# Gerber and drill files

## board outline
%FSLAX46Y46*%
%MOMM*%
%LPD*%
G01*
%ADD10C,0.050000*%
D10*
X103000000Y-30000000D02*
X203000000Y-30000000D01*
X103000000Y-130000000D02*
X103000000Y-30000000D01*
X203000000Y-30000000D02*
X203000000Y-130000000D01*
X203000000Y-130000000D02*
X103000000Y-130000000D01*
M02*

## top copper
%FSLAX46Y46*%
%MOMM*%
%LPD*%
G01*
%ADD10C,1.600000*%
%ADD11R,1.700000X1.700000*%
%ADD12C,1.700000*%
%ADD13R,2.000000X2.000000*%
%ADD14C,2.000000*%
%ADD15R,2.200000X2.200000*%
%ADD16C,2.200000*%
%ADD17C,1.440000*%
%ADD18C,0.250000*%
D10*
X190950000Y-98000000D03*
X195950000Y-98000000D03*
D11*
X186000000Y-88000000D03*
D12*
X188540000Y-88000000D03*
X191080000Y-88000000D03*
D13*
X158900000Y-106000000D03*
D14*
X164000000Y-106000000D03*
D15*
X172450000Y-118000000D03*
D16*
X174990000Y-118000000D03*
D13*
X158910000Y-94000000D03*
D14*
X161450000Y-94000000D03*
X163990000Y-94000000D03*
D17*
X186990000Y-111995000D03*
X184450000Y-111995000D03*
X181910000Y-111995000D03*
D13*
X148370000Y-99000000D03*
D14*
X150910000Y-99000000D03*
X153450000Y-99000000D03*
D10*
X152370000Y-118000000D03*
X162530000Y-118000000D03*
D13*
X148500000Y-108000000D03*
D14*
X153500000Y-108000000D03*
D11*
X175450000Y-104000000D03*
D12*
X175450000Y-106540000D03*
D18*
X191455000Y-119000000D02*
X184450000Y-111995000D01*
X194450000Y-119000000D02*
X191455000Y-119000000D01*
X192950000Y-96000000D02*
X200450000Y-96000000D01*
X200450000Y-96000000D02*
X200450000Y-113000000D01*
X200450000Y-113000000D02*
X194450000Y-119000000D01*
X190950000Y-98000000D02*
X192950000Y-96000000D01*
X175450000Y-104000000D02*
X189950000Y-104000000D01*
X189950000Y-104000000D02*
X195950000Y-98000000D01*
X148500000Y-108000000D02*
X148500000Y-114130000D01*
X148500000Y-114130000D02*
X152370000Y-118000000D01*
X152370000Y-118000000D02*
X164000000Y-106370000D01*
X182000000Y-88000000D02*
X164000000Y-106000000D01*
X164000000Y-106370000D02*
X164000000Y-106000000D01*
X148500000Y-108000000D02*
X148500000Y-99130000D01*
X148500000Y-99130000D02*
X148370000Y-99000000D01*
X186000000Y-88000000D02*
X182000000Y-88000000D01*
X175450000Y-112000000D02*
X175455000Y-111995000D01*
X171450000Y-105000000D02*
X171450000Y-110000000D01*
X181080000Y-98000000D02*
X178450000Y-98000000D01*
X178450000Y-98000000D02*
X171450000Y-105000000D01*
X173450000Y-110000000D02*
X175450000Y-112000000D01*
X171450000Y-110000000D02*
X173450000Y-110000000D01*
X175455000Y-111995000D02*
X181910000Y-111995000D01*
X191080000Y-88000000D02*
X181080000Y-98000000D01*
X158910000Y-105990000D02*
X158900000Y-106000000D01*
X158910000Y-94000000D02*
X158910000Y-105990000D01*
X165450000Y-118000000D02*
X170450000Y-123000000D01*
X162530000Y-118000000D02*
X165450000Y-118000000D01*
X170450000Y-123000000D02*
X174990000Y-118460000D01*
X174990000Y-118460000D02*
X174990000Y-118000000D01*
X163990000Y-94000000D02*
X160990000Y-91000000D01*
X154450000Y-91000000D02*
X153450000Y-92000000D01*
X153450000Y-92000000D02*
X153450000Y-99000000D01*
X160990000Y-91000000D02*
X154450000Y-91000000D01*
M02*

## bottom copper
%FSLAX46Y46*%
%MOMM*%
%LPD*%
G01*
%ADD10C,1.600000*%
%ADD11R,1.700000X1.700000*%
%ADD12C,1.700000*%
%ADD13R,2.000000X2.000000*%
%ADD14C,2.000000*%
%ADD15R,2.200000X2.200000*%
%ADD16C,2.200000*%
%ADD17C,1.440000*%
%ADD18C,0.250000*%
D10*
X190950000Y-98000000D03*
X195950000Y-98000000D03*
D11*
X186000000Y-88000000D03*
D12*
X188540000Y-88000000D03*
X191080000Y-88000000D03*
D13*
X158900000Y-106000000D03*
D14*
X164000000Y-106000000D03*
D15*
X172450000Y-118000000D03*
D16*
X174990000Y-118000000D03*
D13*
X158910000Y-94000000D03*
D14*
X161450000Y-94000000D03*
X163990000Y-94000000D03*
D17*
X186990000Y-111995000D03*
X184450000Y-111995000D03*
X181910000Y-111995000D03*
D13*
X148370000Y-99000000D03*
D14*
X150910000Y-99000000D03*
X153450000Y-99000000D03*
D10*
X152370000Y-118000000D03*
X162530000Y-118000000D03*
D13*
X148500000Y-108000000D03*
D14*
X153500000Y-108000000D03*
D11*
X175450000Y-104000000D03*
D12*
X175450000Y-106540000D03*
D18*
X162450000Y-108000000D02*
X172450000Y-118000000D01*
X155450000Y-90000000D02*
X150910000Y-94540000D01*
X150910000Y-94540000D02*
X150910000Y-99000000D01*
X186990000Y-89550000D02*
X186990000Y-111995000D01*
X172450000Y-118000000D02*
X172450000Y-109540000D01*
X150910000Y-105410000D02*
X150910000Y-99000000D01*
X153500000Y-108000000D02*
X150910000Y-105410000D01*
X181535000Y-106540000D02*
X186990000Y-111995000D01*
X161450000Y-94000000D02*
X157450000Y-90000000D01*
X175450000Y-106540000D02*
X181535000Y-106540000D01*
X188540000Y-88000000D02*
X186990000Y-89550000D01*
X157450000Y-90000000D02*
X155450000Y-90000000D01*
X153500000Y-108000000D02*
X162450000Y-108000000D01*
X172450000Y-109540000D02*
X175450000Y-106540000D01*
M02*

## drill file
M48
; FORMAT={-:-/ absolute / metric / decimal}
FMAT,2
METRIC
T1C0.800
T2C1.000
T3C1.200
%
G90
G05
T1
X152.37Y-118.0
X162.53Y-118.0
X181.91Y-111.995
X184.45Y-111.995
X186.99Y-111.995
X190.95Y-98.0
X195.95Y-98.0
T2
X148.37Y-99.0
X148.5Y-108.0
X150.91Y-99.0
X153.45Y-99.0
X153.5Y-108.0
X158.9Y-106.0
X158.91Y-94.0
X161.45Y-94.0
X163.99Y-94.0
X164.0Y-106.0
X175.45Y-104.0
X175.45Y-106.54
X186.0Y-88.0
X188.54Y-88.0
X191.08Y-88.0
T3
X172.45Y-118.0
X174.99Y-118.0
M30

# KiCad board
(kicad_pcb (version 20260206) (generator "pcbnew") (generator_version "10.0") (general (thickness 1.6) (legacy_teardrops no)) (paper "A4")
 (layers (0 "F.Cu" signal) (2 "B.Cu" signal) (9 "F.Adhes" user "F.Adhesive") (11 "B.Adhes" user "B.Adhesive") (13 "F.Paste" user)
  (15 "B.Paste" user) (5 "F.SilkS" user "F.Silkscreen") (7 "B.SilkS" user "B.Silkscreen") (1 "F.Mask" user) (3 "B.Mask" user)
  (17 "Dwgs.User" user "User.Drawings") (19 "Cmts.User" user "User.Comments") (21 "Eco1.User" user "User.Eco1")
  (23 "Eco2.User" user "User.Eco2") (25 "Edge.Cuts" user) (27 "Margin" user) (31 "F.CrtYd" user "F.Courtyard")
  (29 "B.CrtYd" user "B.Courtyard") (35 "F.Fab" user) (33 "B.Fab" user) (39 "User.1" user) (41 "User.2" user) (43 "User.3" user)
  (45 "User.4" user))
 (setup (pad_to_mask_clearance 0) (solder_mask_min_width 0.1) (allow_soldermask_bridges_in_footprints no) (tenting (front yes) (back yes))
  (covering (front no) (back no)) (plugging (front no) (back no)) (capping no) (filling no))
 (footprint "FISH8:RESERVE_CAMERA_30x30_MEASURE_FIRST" (layer "F.Cu") (at 109.5 35.5)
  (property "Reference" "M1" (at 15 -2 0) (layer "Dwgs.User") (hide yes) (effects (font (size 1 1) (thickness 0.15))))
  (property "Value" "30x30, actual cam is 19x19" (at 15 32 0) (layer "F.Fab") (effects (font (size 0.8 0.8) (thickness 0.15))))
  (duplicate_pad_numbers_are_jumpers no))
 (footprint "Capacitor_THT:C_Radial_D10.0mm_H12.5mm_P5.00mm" (layer "F.Cu") (at 190.95 98)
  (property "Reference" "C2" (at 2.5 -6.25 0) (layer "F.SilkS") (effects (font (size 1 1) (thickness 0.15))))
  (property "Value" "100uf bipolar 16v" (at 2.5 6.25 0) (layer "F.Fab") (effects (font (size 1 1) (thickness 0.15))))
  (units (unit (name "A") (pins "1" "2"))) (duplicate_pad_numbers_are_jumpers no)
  (pad "1" thru_hole circle (at 0 0) (size 1.6 1.6) (drill 0.8) (layers "*.Cu" "*.Mask") (remove_unused_layers no) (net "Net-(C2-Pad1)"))
  (pad "2" thru_hole circle (at 5 0) (size 1.6 1.6) (drill 0.8) (layers "*.Cu" "*.Mask") (remove_unused_layers no) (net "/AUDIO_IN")))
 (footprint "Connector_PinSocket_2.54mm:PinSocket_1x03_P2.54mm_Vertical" (layer "F.Cu") (at 186 88 90)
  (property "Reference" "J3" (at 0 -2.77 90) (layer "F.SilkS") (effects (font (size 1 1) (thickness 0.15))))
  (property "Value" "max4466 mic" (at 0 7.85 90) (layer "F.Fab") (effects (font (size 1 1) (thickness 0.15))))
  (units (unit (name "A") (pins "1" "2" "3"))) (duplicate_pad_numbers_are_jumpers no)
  (pad "1" thru_hole rect (at 0 0 90) (size 1.7 1.7) (drill 1) (layers "*.Cu" "*.Mask") (remove_unused_layers no) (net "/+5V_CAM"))
  (pad "2" thru_hole circle (at 0 2.54 90) (size 1.7 1.7) (drill 1) (layers "*.Cu" "*.Mask") (remove_unused_layers no) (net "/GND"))
  (pad "3" thru_hole circle (at 0 5.08 90) (size 1.7 1.7) (drill 1) (layers "*.Cu" "*.Mask") (remove_unused_layers no) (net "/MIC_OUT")))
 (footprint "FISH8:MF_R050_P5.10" (layer "F.Cu") (at 158.9 106)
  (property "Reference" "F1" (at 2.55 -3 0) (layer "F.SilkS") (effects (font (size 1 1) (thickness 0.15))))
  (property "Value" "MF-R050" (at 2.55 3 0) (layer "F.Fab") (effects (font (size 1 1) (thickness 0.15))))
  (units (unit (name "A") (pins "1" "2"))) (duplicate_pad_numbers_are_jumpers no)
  (pad "1" thru_hole rect (at 0 0) (size 2 2) (drill 1) (layers "*.Cu" "*.Mask") (remove_unused_layers no) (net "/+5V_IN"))
  (pad "2" thru_hole circle (at 5.1 0) (size 2 2) (drill 1) (layers "*.Cu" "*.Mask") (remove_unused_layers no) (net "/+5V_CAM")))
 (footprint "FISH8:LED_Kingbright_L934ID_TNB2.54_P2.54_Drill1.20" (layer "F.Cu") (at 172.45 118)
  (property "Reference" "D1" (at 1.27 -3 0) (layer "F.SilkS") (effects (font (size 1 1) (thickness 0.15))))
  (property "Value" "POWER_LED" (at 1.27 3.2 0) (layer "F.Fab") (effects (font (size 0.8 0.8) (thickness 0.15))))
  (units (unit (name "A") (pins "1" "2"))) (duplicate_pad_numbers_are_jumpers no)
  (pad "1" thru_hole rect (at 0 0) (size 2.2 2.2) (drill 1.2) (layers "*.Cu" "*.Mask") (remove_unused_layers no) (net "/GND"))
  (pad "2" thru_hole circle (at 2.54 0) (size 2.2 2.2) (drill 1.2) (layers "*.Cu" "*.Mask") (remove_unused_layers no) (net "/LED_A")))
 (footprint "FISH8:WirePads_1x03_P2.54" (layer "F.Cu") (at 158.91 94)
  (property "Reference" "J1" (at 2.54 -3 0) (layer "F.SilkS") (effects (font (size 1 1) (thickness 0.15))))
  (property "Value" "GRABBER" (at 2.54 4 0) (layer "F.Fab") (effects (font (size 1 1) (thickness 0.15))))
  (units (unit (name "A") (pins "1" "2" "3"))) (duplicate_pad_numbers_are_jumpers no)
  (pad "1" thru_hole rect (at 0 0) (size 2 2) (drill 1) (layers "*.Cu" "*.Mask") (remove_unused_layers no) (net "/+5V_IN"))
  (pad "2" thru_hole circle (at 2.54 0) (size 2 2) (drill 1) (layers "*.Cu" "*.Mask") (remove_unused_layers no) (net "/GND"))
  (pad "3" thru_hole circle (at 5.08 0) (size 2 2) (drill 1) (layers "*.Cu" "*.Mask") (remove_unused_layers no) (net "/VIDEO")))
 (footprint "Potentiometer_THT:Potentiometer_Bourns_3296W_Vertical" (layer "F.Cu") (at 186.99 111.995)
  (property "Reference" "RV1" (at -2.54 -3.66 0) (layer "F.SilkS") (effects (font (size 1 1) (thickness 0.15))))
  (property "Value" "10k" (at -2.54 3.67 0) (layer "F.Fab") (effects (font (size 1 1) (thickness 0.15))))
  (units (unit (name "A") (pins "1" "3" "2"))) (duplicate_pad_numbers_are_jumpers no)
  (pad "1" thru_hole circle (at 0 0) (size 1.44 1.44) (drill 0.8) (layers "*.Cu" "*.Mask") (remove_unused_layers no) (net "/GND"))
  (pad "2" thru_hole circle (at -2.54 0) (size 1.44 1.44) (drill 0.8) (layers "*.Cu" "*.Mask") (remove_unused_layers no)
   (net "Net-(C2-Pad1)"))
  (pad "3" thru_hole circle (at -5.08 0) (size 1.44 1.44) (drill 0.8) (layers "*.Cu" "*.Mask") (remove_unused_layers no) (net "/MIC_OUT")))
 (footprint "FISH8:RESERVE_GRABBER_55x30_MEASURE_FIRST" (layer "F.Cu") (at 144.5 35.5)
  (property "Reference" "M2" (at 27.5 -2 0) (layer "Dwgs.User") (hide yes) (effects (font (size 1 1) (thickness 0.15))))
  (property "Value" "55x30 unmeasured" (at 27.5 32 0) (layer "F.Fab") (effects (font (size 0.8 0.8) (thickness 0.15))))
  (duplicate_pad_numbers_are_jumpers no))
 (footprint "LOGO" (layer "F.Cu") (at 123 79)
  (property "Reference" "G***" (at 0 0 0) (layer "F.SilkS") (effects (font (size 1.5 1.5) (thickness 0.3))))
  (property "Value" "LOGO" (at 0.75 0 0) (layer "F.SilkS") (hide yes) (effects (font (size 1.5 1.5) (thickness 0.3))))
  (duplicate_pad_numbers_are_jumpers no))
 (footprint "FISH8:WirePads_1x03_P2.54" (layer "F.Cu") (at 148.37 99)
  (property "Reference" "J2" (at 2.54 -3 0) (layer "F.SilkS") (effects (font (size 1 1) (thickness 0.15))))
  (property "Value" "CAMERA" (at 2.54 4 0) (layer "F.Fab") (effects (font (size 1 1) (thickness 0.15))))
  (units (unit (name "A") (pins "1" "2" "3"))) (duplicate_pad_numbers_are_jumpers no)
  (pad "1" thru_hole rect (at 0 0) (size 2 2) (drill 1) (layers "*.Cu" "*.Mask") (remove_unused_layers no) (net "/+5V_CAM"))
  (pad "2" thru_hole circle (at 2.54 0) (size 2 2) (drill 1) (layers "*.Cu" "*.Mask") (remove_unused_layers no) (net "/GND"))
  (pad "3" thru_hole circle (at 5.08 0) (size 2 2) (drill 1) (layers "*.Cu" "*.Mask") (remove_unused_layers no) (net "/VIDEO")))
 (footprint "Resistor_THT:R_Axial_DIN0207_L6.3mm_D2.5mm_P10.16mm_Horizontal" (layer "F.Cu") (at 152.37 118)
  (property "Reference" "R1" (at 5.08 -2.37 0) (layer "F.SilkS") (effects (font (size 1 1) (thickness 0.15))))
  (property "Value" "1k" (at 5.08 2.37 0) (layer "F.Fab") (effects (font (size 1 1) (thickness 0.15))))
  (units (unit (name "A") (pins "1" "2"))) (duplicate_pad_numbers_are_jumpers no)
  (pad "1" thru_hole circle (at 0 0) (size 1.6 1.6) (drill 0.8) (layers "*.Cu" "*.Mask") (remove_unused_layers no) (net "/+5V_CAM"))
  (pad "2" thru_hole circle (at 10.16 0) (size 1.6 1.6) (drill 0.8) (layers "*.Cu" "*.Mask") (remove_unused_layers no) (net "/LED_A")))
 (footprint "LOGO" (layer "F.Cu") (at 148 78)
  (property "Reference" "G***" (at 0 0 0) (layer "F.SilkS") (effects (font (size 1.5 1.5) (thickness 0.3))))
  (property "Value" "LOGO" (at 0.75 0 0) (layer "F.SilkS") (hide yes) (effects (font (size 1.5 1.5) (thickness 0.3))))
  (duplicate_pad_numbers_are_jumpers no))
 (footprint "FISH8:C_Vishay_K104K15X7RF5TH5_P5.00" (layer "F.Cu") (at 148.5 108)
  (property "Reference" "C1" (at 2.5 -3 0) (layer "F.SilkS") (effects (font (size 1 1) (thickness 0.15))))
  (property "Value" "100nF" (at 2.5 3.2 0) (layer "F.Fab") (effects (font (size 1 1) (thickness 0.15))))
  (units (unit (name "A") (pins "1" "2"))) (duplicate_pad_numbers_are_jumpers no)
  (pad "1" thru_hole rect (at 0 0) (size 2 2) (drill 1) (layers "*.Cu" "*.Mask") (remove_unused_layers no) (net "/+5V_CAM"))
  (pad "2" thru_hole circle (at 5 0) (size 2 2) (drill 1) (layers "*.Cu" "*.Mask") (remove_unused_layers no) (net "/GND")))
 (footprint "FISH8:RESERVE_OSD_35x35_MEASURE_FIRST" (layer "F.Cu") (at 108 90)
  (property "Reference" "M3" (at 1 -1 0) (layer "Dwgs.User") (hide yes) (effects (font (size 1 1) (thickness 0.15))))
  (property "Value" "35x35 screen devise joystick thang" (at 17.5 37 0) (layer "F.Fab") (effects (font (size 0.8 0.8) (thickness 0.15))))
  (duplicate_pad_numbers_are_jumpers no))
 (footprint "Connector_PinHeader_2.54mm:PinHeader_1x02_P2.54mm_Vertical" (layer "F.Cu") (at 175.45 104)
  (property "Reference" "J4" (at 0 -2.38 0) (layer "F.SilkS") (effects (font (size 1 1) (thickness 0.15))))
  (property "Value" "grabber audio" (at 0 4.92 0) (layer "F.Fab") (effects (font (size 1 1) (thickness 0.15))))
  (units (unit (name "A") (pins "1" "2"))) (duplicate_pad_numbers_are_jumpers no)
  (pad "1" thru_hole rect (at 0 0) (size 1.7 1.7) (drill 1) (layers "*.Cu" "*.Mask") (remove_unused_layers no) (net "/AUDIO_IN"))
  (pad "2" thru_hole circle (at 0 2.54) (size 1.7 1.7) (drill 1) (layers "*.Cu" "*.Mask") (remove_unused_layers no) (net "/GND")))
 (gr_line (start 103 30) (end 203 30) (stroke (width 0.05) (type default)) (layer "Edge.Cuts"))
 (gr_line (start 103 130) (end 103 30) (stroke (width 0.05) (type default)) (layer "Edge.Cuts"))
 (gr_line (start 203 30) (end 203 130) (stroke (width 0.05) (type default)) (layer "Edge.Cuts"))
 (gr_line (start 203 130) (end 103 130) (stroke (width 0.05) (type default)) (layer "Edge.Cuts"))
 (segment (start 191.455 119) (end 184.45 111.995) (width 0.25) (layer "F.Cu") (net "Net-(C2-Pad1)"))
 (segment (start 194.45 119) (end 191.455 119) (width 0.25) (layer "F.Cu") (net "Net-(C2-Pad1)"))
 (segment (start 192.95 96) (end 200.45 96) (width 0.25) (layer "F.Cu") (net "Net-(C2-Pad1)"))
 (segment (start 200.45 96) (end 200.45 113) (width 0.25) (layer "F.Cu") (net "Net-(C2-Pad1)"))
 (segment (start 200.45 113) (end 194.45 119) (width 0.25) (layer "F.Cu") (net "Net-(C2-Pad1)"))
 (segment (start 190.95 98) (end 192.95 96) (width 0.25) (layer "F.Cu") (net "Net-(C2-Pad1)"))
 (segment (start 175.45 104) (end 189.95 104) (width 0.25) (layer "F.Cu") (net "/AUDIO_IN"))
 (segment (start 189.95 104) (end 195.95 98) (width 0.25) (layer "F.Cu") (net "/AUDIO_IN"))
 (segment (start 148.5 108) (end 148.5 114.13) (width 0.25) (layer "F.Cu") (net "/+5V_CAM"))
 (segment (start 148.5 114.13) (end 152.37 118) (width 0.25) (layer "F.Cu") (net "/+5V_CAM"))
 (segment (start 152.37 118) (end 164 106.37) (width 0.25) (layer "F.Cu") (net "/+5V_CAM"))
 (segment (start 182 88) (end 164 106) (width 0.25) (layer "F.Cu") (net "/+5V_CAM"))
 (segment (start 164 106.37) (end 164 106) (width 0.25) (layer "F.Cu") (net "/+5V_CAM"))
 (segment (start 148.5 108) (end 148.5 99.13) (width 0.25) (layer "F.Cu") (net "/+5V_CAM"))
 (segment (start 148.5 99.13) (end 148.37 99) (width 0.25) (layer "F.Cu") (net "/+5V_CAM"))
 (segment (start 186 88) (end 182 88) (width 0.25) (layer "F.Cu") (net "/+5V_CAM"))
 (segment (start 162.45 108) (end 172.45 118) (width 0.25) (layer "B.Cu") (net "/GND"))
 (segment (start 155.45 90) (end 150.91 94.54) (width 0.25) (layer "B.Cu") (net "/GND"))
 (segment (start 150.91 94.54) (end 150.91 99) (width 0.25) (layer "B.Cu") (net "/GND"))
 (segment (start 186.99 89.55) (end 186.99 111.995) (width 0.25) (layer "B.Cu") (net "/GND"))
 (segment (start 172.45 118) (end 172.45 109.54) (width 0.25) (layer "B.Cu") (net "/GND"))
 (segment (start 150.91 105.41) (end 150.91 99) (width 0.25) (layer "B.Cu") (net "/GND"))
 (segment (start 153.5 108) (end 150.91 105.41) (width 0.25) (layer "B.Cu") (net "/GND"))
 (segment (start 181.535 106.54) (end 186.99 111.995) (width 0.25) (layer "B.Cu") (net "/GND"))
 (segment (start 161.45 94) (end 157.45 90) (width 0.25) (layer "B.Cu") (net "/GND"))
 (segment (start 175.45 106.54) (end 181.535 106.54) (width 0.25) (layer "B.Cu") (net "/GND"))
 (segment (start 188.54 88) (end 186.99 89.55) (width 0.25) (layer "B.Cu") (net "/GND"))
 (segment (start 157.45 90) (end 155.45 90) (width 0.25) (layer "B.Cu") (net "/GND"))
 (segment (start 153.5 108) (end 162.45 108) (width 0.25) (layer "B.Cu") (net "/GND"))
 (segment (start 172.45 109.54) (end 175.45 106.54) (width 0.25) (layer "B.Cu") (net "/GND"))
 (segment (start 175.45 112) (end 175.455 111.995) (width 0.25) (layer "F.Cu") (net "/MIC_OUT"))
 (segment (start 171.45 105) (end 171.45 110) (width 0.25) (layer "F.Cu") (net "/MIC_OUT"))
 (segment (start 181.08 98) (end 178.45 98) (width 0.25) (layer "F.Cu") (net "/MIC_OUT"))
 (segment (start 178.45 98) (end 171.45 105) (width 0.25) (layer "F.Cu") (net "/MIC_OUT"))
 (segment (start 173.45 110) (end 175.45 112) (width 0.25) (layer "F.Cu") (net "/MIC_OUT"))
 (segment (start 171.45 110) (end 173.45 110) (width 0.25) (layer "F.Cu") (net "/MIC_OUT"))
 (segment (start 175.455 111.995) (end 181.91 111.995) (width 0.25) (layer "F.Cu") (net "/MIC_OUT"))
 (segment (start 191.08 88) (end 181.08 98) (width 0.25) (layer "F.Cu") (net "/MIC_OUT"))
 (segment (start 158.91 105.99) (end 158.9 106) (width 0.25) (layer "F.Cu") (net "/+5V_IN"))
 (segment (start 158.91 94) (end 158.91 105.99) (width 0.25) (layer "F.Cu") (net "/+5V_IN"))
 (segment (start 165.45 118) (end 170.45 123) (width 0.25) (layer "F.Cu") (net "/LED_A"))
 (segment (start 162.53 118) (end 165.45 118) (width 0.25) (layer "F.Cu") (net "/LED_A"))
 (segment (start 170.45 123) (end 174.99 118.46) (width 0.25) (layer "F.Cu") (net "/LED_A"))
 (segment (start 174.99 118.46) (end 174.99 118) (width 0.25) (layer "F.Cu") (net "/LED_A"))
 (segment (start 163.99 94) (end 160.99 91) (width 0.25) (layer "F.Cu") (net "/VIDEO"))
 (segment (start 154.45 91) (end 153.45 92) (width 0.25) (layer "F.Cu") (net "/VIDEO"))
 (segment (start 153.45 92) (end 153.45 99) (width 0.25) (layer "F.Cu") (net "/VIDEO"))
 (segment (start 160.99 91) (end 154.45 91) (width 0.25) (layer "F.Cu") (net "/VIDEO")))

